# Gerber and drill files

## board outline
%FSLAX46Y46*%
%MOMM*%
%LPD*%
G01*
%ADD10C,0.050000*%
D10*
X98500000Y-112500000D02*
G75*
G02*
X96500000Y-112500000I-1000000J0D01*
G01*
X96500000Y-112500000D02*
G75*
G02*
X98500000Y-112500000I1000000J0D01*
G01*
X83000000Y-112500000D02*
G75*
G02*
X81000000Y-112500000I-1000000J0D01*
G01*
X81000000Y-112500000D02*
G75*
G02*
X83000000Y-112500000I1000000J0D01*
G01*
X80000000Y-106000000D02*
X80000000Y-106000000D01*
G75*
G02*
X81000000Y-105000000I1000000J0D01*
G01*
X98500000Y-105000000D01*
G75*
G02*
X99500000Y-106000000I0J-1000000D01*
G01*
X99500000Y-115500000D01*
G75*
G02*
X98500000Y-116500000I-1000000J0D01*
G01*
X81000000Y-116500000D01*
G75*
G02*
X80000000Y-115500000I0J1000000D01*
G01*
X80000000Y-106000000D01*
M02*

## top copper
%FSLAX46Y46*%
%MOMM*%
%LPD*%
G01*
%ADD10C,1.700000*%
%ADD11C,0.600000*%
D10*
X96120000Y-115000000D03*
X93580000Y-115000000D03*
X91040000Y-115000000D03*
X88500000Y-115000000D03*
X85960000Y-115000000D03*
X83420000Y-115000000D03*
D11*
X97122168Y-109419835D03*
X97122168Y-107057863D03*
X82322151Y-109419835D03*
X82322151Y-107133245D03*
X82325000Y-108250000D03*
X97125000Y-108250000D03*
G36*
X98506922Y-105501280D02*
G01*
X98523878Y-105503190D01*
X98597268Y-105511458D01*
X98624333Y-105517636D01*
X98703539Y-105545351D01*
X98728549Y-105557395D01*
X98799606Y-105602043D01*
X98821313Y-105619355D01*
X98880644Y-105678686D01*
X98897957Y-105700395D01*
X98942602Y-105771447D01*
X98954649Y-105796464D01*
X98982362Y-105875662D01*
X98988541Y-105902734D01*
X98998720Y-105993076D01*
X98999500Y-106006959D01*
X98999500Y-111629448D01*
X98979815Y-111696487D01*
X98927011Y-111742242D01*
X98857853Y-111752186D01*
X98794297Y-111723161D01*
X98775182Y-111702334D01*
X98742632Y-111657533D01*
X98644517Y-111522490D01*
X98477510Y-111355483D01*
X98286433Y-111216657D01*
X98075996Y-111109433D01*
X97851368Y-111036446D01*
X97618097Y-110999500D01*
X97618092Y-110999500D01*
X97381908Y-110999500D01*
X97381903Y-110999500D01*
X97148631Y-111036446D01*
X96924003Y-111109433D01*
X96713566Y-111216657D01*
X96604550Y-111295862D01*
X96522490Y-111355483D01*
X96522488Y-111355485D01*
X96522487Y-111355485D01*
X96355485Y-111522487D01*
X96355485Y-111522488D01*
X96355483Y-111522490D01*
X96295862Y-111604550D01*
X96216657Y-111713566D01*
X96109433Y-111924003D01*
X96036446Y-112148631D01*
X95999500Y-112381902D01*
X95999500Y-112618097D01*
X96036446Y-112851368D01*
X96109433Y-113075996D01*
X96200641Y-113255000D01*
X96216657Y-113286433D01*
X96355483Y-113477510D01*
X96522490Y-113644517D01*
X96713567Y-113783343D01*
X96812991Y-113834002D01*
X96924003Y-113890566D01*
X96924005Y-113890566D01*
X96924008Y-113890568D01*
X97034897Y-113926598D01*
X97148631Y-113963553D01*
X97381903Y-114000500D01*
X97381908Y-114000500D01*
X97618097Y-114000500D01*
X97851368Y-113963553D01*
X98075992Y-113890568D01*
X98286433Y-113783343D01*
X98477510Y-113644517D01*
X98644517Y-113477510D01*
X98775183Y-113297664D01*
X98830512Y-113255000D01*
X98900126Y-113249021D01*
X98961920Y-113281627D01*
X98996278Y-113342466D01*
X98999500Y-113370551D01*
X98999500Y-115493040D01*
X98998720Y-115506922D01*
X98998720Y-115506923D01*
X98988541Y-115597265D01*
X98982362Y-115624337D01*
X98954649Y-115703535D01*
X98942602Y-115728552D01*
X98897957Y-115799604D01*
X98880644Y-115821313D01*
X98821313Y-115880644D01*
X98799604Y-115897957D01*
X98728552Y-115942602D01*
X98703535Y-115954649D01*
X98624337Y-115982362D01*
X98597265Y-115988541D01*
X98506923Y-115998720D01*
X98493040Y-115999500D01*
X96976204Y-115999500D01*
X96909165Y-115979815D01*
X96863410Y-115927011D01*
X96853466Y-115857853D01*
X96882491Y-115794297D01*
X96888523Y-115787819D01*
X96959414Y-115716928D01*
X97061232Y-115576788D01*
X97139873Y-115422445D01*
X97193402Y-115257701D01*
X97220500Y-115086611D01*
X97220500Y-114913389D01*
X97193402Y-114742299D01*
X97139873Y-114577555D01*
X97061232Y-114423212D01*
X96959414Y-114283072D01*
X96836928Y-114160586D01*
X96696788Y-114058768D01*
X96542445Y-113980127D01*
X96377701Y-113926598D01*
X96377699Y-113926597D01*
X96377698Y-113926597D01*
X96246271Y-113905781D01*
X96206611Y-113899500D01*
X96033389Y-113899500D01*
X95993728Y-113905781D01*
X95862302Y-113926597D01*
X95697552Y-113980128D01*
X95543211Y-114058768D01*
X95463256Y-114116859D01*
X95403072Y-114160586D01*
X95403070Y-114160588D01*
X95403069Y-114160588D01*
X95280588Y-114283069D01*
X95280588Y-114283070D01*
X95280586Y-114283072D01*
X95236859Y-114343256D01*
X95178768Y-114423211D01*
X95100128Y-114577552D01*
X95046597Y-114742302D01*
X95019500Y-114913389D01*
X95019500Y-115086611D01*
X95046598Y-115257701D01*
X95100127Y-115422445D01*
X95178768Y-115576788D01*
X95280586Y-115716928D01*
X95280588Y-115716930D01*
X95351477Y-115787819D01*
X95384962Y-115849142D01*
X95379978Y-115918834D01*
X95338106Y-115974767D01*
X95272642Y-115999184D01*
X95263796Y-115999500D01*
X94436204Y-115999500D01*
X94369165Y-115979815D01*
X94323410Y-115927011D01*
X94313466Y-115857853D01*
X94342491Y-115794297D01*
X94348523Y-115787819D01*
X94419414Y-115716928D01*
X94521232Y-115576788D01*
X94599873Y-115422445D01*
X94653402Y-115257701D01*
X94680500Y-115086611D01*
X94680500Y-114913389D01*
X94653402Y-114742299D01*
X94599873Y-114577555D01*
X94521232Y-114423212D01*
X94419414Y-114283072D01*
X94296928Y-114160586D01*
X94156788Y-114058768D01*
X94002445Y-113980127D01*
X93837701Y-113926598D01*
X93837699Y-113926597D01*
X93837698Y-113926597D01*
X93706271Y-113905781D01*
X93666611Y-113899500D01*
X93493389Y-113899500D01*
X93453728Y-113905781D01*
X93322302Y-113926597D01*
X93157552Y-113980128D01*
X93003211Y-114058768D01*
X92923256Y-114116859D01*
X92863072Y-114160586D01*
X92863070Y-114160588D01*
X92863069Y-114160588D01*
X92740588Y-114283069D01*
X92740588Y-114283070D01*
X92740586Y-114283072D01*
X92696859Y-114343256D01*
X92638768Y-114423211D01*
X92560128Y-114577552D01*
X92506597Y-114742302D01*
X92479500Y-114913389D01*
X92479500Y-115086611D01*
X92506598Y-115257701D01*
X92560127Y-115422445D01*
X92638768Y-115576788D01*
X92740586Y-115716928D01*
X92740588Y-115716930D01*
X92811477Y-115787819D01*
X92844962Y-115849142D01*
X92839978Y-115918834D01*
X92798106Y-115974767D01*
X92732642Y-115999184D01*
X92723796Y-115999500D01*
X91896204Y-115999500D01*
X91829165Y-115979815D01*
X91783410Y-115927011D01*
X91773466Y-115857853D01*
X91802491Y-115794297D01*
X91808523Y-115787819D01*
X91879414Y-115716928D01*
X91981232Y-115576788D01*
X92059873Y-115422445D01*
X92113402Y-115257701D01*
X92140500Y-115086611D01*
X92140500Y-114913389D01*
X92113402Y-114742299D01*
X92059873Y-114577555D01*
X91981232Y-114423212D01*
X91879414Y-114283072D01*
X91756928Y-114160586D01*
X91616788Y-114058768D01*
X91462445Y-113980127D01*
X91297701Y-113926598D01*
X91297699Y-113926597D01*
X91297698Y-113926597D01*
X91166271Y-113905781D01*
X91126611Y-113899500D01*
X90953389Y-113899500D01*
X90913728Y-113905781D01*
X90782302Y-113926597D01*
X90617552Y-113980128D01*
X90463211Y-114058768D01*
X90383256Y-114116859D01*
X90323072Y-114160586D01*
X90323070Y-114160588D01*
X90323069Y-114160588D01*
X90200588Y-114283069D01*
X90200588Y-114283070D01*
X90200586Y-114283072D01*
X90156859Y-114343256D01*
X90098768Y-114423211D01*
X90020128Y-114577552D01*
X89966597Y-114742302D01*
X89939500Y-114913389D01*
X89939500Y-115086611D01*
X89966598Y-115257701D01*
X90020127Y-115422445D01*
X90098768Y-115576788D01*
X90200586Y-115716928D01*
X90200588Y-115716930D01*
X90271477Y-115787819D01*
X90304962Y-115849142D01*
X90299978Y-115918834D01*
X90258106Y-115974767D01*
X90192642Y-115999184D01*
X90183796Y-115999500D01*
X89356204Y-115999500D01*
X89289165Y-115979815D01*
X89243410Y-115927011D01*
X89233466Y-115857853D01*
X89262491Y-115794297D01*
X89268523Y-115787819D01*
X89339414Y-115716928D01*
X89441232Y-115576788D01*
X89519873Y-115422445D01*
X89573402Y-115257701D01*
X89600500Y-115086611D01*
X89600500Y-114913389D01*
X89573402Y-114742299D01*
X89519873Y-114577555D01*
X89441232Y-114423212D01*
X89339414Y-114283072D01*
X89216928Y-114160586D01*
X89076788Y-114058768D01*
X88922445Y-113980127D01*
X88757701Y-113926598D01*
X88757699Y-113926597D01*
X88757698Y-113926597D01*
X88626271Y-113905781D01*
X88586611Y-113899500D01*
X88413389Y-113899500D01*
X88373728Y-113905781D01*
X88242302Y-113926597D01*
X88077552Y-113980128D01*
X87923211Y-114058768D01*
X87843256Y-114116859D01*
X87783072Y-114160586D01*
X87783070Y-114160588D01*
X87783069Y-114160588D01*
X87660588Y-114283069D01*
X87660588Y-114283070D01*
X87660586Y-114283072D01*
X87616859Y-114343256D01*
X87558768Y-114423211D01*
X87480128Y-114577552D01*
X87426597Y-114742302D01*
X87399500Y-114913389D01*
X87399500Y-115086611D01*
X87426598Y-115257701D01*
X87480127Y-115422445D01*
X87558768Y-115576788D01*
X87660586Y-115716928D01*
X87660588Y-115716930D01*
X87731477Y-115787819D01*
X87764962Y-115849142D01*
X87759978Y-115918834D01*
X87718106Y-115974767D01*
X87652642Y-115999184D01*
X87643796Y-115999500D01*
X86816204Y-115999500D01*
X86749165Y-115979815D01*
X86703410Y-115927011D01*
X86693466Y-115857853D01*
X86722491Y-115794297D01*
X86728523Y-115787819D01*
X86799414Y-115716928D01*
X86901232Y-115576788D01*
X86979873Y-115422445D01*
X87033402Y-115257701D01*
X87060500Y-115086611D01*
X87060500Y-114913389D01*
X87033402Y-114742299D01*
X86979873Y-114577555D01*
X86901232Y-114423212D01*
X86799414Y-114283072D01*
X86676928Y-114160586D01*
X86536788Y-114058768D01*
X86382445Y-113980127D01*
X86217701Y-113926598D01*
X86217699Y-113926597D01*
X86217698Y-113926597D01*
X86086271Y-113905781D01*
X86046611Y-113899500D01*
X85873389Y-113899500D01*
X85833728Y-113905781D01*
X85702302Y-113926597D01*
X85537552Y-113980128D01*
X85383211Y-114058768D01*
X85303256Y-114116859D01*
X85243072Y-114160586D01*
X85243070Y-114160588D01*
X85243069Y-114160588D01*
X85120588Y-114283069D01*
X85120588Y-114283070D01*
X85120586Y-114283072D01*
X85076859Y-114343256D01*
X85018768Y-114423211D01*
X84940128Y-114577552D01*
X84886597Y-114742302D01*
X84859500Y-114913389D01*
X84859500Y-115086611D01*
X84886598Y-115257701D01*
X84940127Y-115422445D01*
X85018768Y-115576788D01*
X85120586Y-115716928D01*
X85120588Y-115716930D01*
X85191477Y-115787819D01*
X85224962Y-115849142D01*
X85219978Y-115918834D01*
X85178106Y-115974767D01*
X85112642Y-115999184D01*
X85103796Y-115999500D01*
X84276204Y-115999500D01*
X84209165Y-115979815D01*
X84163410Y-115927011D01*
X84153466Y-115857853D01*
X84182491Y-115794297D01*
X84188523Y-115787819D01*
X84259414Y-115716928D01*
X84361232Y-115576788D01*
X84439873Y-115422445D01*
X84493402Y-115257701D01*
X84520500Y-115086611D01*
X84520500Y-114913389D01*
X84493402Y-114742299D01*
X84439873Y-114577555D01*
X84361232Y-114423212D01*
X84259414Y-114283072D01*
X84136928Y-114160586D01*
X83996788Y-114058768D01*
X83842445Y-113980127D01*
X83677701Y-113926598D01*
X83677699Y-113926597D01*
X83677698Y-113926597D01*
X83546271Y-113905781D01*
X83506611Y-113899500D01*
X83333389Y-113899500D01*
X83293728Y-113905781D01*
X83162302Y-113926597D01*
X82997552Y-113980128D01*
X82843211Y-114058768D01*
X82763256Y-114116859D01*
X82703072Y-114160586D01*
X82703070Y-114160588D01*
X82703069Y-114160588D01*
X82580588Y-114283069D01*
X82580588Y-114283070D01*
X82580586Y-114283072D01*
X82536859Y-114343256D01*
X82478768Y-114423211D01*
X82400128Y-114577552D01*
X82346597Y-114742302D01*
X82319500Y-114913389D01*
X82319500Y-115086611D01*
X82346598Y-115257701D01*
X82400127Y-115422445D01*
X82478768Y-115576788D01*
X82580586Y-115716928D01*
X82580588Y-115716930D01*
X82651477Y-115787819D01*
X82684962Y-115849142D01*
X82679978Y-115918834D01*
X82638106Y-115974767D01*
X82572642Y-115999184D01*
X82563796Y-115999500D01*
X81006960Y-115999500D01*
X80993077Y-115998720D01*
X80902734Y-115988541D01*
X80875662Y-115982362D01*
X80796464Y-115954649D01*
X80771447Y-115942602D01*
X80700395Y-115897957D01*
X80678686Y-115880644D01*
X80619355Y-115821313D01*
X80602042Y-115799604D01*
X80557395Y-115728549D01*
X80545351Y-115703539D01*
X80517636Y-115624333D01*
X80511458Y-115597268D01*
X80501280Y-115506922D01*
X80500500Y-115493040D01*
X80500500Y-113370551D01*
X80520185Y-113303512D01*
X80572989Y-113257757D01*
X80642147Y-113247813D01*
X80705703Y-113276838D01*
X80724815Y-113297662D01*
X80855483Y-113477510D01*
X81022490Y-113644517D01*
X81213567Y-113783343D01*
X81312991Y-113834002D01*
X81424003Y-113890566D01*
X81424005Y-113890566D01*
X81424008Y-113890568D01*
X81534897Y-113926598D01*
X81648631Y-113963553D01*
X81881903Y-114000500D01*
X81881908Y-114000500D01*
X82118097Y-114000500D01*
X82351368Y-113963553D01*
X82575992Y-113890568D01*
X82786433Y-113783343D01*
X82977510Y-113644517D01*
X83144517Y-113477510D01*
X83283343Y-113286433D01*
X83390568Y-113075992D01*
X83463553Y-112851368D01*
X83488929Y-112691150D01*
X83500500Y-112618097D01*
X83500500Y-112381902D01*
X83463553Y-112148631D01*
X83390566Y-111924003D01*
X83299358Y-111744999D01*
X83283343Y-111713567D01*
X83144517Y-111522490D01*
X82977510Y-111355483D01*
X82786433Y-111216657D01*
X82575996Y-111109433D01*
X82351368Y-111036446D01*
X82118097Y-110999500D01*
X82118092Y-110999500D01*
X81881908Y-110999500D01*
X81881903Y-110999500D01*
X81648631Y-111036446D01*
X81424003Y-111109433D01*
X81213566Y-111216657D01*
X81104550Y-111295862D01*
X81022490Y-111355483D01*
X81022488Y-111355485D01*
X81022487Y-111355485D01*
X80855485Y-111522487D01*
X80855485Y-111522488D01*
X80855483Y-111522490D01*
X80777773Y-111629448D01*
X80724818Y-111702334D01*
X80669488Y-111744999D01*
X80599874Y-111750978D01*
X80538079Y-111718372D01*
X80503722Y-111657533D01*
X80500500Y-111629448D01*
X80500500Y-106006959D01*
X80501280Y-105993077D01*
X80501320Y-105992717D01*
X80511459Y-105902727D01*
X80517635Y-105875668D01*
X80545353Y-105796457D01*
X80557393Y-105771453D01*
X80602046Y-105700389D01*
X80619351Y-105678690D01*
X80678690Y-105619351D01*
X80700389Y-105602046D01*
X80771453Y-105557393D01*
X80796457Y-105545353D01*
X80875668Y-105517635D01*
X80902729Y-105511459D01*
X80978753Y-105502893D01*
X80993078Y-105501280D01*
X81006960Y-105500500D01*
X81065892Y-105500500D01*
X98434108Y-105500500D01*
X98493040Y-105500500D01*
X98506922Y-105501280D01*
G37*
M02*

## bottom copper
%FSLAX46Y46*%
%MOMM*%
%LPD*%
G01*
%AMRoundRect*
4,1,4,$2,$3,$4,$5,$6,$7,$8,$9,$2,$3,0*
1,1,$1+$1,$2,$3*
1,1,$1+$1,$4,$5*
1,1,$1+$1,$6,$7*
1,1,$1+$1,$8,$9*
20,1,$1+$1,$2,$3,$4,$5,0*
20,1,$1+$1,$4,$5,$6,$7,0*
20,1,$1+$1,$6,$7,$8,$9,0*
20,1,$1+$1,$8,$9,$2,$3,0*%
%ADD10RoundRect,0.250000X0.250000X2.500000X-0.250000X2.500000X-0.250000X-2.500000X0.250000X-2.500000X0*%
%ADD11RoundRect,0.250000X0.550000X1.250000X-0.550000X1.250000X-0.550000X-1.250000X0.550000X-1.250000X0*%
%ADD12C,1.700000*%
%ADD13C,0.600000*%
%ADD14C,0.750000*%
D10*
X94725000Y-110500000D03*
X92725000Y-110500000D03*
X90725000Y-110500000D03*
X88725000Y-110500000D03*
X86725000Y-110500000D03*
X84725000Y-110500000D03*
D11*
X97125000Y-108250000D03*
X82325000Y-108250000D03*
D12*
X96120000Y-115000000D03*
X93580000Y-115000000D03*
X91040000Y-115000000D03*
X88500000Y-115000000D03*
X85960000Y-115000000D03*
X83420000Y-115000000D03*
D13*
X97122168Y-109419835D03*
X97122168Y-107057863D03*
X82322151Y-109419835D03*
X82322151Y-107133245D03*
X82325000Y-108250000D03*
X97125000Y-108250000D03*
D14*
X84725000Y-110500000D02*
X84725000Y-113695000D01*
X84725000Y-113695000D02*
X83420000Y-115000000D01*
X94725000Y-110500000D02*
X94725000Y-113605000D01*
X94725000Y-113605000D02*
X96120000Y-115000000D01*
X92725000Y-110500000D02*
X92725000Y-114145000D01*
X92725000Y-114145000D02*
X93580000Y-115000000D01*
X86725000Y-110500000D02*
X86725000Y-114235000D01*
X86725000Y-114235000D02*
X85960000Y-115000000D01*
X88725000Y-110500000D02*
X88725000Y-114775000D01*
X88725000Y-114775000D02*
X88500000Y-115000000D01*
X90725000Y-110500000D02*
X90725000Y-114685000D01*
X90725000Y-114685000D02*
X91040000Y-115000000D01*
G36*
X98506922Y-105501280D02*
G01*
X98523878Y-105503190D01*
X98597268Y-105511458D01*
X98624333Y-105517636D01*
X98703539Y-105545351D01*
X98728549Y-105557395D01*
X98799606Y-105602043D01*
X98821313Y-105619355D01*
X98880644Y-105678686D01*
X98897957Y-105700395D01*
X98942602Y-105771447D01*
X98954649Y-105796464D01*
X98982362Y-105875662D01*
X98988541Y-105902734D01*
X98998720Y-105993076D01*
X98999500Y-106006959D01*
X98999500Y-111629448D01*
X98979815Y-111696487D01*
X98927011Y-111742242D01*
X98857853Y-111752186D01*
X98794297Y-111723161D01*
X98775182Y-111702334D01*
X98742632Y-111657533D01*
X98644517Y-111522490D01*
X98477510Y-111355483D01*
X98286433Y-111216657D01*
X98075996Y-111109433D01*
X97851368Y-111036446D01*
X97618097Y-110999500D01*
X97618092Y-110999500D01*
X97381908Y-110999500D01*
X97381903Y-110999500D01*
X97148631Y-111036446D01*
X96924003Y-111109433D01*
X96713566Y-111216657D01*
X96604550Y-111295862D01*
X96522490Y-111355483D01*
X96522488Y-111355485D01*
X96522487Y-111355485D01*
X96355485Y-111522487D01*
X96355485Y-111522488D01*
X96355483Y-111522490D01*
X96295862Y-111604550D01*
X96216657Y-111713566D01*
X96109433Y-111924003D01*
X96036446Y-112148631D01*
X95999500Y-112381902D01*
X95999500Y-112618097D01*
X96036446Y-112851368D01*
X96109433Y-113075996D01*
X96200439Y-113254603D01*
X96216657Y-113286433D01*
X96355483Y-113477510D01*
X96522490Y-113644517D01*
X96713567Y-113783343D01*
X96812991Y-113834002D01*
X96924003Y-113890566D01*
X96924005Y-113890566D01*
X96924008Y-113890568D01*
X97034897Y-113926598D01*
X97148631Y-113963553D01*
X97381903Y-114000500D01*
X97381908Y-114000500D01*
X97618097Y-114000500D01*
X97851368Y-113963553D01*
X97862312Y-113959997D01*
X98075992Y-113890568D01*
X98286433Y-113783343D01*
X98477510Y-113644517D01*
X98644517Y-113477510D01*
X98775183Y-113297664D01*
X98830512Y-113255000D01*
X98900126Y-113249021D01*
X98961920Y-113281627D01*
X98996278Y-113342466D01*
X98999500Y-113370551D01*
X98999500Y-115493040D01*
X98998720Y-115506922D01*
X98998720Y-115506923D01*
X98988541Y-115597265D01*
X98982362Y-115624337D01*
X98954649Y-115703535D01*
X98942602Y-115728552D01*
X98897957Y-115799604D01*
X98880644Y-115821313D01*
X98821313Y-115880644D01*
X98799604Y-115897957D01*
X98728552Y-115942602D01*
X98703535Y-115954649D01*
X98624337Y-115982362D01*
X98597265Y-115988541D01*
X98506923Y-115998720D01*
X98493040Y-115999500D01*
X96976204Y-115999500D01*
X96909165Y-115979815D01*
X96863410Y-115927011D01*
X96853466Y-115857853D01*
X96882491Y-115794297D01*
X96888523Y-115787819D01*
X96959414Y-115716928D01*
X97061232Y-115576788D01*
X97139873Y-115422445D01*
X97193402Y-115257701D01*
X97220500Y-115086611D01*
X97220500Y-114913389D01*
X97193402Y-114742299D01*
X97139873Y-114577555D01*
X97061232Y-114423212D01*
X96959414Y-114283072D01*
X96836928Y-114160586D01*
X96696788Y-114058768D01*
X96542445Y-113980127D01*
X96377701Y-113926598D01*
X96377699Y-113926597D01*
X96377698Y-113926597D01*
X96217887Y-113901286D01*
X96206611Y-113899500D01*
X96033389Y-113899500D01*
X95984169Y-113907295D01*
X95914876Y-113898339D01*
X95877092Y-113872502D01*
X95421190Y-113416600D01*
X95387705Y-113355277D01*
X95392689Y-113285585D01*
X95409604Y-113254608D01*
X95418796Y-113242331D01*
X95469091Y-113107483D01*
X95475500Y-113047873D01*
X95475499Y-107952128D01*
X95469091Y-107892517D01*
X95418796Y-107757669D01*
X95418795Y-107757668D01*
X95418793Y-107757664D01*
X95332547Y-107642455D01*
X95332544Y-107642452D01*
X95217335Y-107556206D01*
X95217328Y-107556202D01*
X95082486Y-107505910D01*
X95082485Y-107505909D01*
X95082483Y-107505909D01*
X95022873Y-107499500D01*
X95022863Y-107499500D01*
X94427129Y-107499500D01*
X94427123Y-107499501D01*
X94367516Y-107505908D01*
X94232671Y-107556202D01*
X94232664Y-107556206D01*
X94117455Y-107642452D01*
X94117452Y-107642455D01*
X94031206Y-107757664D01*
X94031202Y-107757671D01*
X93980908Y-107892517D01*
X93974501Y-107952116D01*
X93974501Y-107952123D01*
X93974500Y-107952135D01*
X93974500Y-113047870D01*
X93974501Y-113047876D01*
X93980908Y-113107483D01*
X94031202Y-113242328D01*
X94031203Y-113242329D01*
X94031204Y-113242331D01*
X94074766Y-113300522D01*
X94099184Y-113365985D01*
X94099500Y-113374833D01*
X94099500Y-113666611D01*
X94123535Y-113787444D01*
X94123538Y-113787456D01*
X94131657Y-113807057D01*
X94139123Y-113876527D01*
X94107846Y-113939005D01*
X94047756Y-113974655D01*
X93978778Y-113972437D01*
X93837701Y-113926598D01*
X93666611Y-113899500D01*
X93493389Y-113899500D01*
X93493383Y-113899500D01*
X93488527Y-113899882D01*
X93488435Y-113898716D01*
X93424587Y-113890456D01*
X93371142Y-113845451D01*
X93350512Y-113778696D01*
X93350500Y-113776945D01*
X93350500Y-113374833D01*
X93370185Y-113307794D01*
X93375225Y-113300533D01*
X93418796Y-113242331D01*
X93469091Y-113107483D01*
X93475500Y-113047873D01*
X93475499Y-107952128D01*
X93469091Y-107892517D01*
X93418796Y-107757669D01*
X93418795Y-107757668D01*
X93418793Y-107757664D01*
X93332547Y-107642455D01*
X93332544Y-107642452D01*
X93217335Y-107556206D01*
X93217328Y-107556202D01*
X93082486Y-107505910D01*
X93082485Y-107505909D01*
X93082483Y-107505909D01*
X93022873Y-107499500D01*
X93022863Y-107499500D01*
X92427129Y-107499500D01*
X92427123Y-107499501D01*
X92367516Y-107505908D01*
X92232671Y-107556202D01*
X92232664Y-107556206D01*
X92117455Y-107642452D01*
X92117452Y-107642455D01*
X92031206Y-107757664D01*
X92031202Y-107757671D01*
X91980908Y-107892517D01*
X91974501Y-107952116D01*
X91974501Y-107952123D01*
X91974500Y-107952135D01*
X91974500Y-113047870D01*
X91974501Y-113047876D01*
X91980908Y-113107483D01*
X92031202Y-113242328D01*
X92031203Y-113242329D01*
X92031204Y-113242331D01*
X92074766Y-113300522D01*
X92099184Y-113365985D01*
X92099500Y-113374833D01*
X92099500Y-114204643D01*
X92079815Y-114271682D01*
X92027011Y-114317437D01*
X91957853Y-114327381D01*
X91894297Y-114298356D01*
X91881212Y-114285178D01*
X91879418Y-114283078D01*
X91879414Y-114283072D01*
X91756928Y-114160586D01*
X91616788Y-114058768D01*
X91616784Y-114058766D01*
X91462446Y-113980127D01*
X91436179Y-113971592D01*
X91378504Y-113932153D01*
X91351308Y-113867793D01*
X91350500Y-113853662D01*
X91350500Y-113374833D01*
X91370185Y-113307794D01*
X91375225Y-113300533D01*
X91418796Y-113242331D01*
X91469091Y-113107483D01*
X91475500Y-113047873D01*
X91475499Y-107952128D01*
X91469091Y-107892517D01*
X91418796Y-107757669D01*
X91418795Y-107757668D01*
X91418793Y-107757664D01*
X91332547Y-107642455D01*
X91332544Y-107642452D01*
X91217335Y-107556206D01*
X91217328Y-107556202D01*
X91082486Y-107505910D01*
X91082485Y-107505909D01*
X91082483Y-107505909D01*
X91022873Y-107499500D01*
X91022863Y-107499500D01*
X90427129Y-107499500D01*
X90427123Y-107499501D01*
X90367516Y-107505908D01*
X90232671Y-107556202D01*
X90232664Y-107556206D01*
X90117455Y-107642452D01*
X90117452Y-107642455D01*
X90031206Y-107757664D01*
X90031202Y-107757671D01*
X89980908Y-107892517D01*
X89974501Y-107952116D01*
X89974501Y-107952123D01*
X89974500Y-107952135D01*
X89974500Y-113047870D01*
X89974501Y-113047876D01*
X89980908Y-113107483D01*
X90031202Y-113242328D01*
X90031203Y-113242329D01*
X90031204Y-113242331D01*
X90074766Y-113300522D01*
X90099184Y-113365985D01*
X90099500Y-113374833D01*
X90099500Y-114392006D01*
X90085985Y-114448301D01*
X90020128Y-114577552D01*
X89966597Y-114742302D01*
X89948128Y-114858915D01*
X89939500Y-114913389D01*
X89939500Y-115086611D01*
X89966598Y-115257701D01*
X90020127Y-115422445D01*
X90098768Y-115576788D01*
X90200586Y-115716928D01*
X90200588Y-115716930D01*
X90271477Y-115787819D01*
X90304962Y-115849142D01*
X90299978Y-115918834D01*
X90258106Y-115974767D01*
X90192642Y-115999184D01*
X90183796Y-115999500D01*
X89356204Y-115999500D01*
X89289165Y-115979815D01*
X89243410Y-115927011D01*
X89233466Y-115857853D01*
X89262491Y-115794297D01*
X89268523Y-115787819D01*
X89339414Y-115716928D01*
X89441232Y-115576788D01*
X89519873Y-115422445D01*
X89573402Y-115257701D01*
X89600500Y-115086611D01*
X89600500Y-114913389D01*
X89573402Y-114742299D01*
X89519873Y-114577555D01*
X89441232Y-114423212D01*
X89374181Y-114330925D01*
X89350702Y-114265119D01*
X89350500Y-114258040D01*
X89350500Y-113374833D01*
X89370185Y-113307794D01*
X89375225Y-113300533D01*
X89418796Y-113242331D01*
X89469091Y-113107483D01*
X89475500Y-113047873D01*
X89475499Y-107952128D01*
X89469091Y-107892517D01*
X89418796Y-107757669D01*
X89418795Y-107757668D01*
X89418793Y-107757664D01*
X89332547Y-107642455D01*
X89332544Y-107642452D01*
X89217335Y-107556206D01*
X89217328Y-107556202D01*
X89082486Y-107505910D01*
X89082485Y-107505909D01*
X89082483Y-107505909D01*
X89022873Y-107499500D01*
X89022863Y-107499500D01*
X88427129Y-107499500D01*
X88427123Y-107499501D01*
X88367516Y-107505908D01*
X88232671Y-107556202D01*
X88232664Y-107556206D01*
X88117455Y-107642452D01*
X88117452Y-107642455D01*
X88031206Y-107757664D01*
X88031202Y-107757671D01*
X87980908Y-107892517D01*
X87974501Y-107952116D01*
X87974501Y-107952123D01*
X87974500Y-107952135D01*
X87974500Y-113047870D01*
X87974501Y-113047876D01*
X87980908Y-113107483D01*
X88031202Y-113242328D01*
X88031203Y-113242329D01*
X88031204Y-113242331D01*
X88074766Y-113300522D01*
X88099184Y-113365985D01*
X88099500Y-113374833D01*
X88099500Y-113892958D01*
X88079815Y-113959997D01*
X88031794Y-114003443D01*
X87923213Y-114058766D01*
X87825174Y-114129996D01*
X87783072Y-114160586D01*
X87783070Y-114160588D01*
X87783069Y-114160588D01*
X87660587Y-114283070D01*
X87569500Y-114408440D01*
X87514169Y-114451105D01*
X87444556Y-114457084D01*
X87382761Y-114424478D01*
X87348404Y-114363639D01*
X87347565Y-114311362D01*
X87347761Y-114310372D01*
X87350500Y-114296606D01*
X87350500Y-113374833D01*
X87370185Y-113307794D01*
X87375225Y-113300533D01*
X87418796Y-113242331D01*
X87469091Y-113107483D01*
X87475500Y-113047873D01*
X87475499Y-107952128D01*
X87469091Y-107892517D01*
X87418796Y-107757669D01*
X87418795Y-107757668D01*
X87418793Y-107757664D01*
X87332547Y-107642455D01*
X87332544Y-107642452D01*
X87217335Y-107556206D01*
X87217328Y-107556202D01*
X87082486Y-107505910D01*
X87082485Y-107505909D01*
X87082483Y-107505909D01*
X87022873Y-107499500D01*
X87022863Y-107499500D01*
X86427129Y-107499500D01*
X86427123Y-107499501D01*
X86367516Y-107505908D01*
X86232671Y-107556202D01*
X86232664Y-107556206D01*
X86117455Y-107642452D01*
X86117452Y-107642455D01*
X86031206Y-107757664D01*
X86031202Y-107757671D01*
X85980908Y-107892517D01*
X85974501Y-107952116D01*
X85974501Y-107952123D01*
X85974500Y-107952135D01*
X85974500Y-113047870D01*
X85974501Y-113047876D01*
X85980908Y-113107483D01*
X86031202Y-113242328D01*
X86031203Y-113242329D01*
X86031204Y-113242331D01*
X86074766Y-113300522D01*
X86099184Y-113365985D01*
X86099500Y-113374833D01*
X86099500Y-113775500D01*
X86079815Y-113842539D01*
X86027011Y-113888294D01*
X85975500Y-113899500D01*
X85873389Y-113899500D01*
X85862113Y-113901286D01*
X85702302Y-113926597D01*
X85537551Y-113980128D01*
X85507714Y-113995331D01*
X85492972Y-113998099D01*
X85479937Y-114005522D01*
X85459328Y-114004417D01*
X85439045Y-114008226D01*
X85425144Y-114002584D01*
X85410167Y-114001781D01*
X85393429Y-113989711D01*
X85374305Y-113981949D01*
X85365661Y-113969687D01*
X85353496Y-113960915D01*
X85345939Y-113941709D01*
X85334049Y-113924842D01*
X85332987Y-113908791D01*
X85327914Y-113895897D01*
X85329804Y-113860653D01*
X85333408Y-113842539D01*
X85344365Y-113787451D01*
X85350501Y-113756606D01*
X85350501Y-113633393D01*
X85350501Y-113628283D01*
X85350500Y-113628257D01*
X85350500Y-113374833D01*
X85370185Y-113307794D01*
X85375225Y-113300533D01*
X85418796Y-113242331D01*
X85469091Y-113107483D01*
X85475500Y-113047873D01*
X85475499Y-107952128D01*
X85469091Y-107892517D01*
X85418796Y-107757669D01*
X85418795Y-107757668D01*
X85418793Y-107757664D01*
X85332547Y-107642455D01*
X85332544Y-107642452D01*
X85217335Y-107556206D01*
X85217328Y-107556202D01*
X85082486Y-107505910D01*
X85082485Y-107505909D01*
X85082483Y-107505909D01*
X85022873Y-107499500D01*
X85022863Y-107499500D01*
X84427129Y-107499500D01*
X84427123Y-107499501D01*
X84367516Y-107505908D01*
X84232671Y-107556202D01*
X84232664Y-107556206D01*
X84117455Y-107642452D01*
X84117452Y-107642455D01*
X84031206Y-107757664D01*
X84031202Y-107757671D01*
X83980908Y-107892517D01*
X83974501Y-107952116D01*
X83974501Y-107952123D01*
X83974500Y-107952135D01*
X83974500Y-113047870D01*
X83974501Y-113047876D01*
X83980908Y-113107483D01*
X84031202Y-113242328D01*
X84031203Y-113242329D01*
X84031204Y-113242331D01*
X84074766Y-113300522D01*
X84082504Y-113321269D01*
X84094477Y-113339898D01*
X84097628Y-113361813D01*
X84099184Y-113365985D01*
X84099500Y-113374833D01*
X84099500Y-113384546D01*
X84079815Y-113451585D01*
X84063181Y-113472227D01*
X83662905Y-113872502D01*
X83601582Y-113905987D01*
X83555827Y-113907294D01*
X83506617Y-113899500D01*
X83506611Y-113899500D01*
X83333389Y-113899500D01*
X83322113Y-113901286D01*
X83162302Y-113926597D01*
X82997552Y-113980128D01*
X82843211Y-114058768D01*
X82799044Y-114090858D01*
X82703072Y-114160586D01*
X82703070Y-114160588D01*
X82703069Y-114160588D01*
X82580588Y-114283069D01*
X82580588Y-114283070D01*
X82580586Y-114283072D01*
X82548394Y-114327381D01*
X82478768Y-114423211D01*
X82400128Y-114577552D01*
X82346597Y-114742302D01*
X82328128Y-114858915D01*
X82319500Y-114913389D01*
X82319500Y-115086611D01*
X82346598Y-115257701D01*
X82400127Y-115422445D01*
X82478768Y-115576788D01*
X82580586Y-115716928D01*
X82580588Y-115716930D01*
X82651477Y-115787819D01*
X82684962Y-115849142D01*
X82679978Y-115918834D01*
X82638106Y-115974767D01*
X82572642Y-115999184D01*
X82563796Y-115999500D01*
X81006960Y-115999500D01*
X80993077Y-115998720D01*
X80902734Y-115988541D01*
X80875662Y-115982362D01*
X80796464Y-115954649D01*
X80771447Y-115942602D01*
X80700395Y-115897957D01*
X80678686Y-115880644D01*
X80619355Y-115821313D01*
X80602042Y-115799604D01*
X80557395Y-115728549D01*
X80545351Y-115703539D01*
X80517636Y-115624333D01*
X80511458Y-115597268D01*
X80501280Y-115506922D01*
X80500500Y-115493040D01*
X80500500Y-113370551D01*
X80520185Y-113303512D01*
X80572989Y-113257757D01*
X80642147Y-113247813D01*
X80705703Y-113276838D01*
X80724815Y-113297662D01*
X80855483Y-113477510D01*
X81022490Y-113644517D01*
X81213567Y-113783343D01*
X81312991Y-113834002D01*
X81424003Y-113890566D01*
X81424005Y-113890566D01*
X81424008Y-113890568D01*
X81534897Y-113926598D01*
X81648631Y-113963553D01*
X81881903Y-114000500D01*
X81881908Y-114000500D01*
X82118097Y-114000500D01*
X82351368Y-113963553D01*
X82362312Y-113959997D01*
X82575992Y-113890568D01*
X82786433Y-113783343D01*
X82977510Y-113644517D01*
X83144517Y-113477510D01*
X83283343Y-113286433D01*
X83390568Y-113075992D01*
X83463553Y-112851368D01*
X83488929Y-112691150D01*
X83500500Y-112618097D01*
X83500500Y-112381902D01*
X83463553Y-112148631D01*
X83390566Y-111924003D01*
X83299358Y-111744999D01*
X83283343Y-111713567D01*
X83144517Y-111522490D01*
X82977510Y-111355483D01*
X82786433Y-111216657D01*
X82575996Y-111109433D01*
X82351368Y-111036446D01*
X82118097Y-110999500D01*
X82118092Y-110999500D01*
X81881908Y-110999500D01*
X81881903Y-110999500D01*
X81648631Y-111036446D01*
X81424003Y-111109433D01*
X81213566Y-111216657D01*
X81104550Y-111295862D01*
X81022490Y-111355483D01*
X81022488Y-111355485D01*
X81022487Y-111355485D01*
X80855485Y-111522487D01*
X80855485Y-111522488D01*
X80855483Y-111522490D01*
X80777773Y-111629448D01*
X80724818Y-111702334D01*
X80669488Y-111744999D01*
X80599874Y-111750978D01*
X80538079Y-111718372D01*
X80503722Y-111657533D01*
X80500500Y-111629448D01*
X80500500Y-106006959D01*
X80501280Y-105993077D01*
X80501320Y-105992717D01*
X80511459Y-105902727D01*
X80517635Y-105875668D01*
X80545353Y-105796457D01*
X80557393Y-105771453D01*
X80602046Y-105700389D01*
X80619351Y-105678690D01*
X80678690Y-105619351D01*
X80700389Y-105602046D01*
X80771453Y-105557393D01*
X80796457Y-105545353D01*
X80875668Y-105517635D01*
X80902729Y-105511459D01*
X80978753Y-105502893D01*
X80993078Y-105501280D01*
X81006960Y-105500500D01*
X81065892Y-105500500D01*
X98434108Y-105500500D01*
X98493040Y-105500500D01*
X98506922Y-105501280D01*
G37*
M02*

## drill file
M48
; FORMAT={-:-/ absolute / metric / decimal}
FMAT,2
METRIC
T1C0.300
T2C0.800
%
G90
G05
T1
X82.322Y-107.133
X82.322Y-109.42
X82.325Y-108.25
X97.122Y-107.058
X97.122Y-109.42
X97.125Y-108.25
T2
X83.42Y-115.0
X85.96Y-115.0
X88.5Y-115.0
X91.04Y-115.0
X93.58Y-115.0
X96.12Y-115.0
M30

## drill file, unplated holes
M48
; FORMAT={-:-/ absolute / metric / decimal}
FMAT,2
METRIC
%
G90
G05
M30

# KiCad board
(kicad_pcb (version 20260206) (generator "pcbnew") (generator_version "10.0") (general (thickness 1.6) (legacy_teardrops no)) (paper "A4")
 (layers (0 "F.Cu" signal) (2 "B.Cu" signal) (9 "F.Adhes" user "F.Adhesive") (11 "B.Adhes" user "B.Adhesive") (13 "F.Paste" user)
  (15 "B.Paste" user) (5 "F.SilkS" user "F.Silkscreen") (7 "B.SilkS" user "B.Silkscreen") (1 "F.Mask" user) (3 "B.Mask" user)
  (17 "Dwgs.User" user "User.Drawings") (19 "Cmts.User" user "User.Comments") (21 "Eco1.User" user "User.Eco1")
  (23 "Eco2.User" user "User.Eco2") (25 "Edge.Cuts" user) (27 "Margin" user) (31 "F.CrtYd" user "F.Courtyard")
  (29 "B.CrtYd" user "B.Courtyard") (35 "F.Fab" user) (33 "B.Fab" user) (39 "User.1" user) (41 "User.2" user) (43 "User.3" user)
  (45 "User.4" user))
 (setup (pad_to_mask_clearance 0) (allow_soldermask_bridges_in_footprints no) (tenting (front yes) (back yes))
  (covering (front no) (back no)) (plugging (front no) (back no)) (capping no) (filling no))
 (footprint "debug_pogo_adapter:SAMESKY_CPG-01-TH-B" (layer "F.Cu") (at 93.58 115)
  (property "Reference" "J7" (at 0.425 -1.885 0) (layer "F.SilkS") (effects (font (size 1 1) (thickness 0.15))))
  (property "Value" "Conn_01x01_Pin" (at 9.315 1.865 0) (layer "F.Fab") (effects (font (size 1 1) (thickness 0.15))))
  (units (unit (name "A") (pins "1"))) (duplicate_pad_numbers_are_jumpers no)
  (pad "1" thru_hole circle (at 0 0) (size 1.7 1.7) (drill 0.8) (layers "*.Cu" "*.Mask") (remove_unused_layers no) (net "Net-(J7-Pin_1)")
   (solder_mask_margin 0.102)))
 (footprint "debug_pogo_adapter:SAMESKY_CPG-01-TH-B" (layer "F.Cu") (at 91.04 115)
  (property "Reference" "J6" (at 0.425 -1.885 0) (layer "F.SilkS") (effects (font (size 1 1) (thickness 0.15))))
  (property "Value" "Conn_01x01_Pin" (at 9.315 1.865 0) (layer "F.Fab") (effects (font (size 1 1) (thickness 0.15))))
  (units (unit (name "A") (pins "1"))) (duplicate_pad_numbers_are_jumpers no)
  (pad "1" thru_hole circle (at 0 0) (size 1.7 1.7) (drill 0.8) (layers "*.Cu" "*.Mask") (remove_unused_layers no) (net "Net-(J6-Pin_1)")
   (solder_mask_margin 0.102)))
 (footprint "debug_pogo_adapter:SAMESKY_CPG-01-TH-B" (layer "F.Cu") (at 85.96 115)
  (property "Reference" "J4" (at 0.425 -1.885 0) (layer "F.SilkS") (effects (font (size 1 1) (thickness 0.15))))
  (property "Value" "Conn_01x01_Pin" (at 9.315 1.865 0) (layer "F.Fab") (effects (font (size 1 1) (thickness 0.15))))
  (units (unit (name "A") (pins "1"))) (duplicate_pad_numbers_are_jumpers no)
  (pad "1" thru_hole circle (at 0 0) (size 1.7 1.7) (drill 0.8) (layers "*.Cu" "*.Mask") (remove_unused_layers no) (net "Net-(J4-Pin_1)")
   (solder_mask_margin 0.102)))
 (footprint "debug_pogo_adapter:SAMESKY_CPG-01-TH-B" (layer "F.Cu") (at 96.12 115)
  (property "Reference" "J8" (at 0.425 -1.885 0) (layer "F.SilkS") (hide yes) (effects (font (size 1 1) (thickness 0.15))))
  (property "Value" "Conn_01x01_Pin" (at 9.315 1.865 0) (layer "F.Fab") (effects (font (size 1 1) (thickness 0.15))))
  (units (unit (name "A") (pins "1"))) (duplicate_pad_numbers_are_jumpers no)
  (pad "1" thru_hole circle (at 0 0) (size 1.7 1.7) (drill 0.8) (layers "*.Cu" "*.Mask") (remove_unused_layers no) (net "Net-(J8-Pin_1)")
   (solder_mask_margin 0.102)))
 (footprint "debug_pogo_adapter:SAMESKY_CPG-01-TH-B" (layer "F.Cu") (at 88.5 115)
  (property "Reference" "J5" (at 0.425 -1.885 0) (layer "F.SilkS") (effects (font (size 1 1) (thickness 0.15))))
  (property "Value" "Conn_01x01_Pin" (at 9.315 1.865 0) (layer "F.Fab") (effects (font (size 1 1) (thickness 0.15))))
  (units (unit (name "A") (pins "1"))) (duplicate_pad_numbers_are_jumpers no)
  (pad "1" thru_hole circle (at 0 0) (size 1.7 1.7) (drill 0.8) (layers "*.Cu" "*.Mask") (remove_unused_layers no) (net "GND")
   (solder_mask_margin 0.102)))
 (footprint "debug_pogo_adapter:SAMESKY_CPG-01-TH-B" (layer "F.Cu") (at 83.42 115)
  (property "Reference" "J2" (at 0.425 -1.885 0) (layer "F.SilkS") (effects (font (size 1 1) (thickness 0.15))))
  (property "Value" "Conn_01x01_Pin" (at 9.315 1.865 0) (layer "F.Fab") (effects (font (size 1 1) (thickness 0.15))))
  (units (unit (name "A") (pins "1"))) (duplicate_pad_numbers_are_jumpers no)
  (pad "1" thru_hole circle (at 0 0) (size 1.7 1.7) (drill 0.8) (layers "*.Cu" "*.Mask") (remove_unused_layers no) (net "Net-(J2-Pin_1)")
   (solder_mask_margin 0.102)))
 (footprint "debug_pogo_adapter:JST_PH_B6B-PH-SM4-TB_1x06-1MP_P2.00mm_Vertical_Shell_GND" (layer "B.Cu") (at 89.725 110 180)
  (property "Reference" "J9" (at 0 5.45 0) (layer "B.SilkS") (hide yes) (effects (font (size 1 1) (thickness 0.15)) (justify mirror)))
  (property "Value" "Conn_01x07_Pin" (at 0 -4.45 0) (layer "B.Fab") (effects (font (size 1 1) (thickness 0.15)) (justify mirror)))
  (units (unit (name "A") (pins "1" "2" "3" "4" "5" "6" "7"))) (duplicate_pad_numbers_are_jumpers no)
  (pad "1" smd roundrect (at -5 -0.5 180) (size 1 5.5) (layers "B.Cu" "B.Mask" "B.Paste") (roundrect_rratio 0.25) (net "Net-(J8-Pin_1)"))
  (pad "2" smd roundrect (at -3 -0.5 180) (size 1 5.5) (layers "B.Cu" "B.Mask" "B.Paste") (roundrect_rratio 0.25) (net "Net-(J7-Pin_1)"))
  (pad "3" smd roundrect (at -1 -0.5 180) (size 1 5.5) (layers "B.Cu" "B.Mask" "B.Paste") (roundrect_rratio 0.25) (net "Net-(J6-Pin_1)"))
  (pad "4" smd roundrect (at 1 -0.5 180) (size 1 5.5) (layers "B.Cu" "B.Mask" "B.Paste") (roundrect_rratio 0.25) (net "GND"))
  (pad "5" smd roundrect (at 3 -0.5 180) (size 1 5.5) (layers "B.Cu" "B.Mask" "B.Paste") (roundrect_rratio 0.25) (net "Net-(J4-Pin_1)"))
  (pad "6" smd roundrect (at 5 -0.5 180) (size 1 5.5) (layers "B.Cu" "B.Mask" "B.Paste") (roundrect_rratio 0.25) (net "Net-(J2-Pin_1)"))
  (pad "7" smd roundrect (at -7.4 1.75 180) (size 1.6 3) (layers "B.Cu" "B.Mask" "B.Paste") (roundrect_rratio 0.15625) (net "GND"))
  (pad "7" smd roundrect (at 7.4 1.75 180) (size 1.6 3) (layers "B.Cu" "B.Mask" "B.Paste") (roundrect_rratio 0.15625) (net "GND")))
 (gr_rect (start 80 105) (end 99.5 116.5) (radius 1) (stroke (width 0.05) (type default)) (fill no) (layer "Edge.Cuts"))
 (gr_circle (center 82 112.5) (end 82 111.5) (stroke (width 0.05) (type default)) (fill no) (layer "Edge.Cuts"))
 (gr_circle (center 97.5 112.5) (end 97.5 111.5) (stroke (width 0.05) (type default)) (fill no) (layer "Edge.Cuts"))
 (segment (start 92.725 114.145) (end 93.58 115) (width 0.75) (layer "B.Cu") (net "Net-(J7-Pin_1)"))
 (segment (start 92.725 110.5) (end 92.725 114.145) (width 0.75) (layer "B.Cu") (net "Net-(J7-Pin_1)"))
 (segment (start 90.725 114.685) (end 91.04 115) (width 0.75) (layer "B.Cu") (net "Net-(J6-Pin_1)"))
 (segment (start 90.725 110.5) (end 90.725 114.685) (width 0.75) (layer "B.Cu") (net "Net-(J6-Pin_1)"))
 (segment (start 86.725 110.5) (end 86.725 114.235) (width 0.75) (layer "B.Cu") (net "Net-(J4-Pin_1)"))
 (segment (start 86.725 114.235) (end 85.96 115) (width 0.75) (layer "B.Cu") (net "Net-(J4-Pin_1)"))
 (segment (start 94.725 113.605) (end 96.12 115) (width 0.75) (layer "B.Cu") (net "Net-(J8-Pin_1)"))
 (segment (start 94.725 110.5) (end 94.725 113.605) (width 0.75) (layer "B.Cu") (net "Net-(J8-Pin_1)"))
 (via (at 82.322151 109.419835) (size 0.6) (drill 0.3) (layers "F.Cu" "B.Cu") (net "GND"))
 (via (at 97.122168 107.057863) (size 0.6) (drill 0.3) (layers "F.Cu" "B.Cu") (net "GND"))
 (via (at 97.125 108.25) (size 0.6) (drill 0.3) (layers "F.Cu" "B.Cu") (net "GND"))
 (via (at 97.122168 109.419835) (size 0.6) (drill 0.3) (layers "F.Cu" "B.Cu") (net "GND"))
 (via (at 82.325 108.25) (size 0.6) (drill 0.3) (layers "F.Cu" "B.Cu") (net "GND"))
 (via (at 82.322151 107.133245) (size 0.6) (drill 0.3) (layers "F.Cu" "B.Cu") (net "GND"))
 (segment (start 88.725 110.5) (end 88.725 114.775) (width 0.75) (layer "B.Cu") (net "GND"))
 (segment (start 88.725 114.775) (end 88.5 115) (width 0.75) (layer "B.Cu") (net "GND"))
 (segment (start 84.725 113.695) (end 83.42 115) (width 0.75) (layer "B.Cu") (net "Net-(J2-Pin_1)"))
 (segment (start 84.725 110.5) (end 84.725 113.695) (width 0.75) (layer "B.Cu") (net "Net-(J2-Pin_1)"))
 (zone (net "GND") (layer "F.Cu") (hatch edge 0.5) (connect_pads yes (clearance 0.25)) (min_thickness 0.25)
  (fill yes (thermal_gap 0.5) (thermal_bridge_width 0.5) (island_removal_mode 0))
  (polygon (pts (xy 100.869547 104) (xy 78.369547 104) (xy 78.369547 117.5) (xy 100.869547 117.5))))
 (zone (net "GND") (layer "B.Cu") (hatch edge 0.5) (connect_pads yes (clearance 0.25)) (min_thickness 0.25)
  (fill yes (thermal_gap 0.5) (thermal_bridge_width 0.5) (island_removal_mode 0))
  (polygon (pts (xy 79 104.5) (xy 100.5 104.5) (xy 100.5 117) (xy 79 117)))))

